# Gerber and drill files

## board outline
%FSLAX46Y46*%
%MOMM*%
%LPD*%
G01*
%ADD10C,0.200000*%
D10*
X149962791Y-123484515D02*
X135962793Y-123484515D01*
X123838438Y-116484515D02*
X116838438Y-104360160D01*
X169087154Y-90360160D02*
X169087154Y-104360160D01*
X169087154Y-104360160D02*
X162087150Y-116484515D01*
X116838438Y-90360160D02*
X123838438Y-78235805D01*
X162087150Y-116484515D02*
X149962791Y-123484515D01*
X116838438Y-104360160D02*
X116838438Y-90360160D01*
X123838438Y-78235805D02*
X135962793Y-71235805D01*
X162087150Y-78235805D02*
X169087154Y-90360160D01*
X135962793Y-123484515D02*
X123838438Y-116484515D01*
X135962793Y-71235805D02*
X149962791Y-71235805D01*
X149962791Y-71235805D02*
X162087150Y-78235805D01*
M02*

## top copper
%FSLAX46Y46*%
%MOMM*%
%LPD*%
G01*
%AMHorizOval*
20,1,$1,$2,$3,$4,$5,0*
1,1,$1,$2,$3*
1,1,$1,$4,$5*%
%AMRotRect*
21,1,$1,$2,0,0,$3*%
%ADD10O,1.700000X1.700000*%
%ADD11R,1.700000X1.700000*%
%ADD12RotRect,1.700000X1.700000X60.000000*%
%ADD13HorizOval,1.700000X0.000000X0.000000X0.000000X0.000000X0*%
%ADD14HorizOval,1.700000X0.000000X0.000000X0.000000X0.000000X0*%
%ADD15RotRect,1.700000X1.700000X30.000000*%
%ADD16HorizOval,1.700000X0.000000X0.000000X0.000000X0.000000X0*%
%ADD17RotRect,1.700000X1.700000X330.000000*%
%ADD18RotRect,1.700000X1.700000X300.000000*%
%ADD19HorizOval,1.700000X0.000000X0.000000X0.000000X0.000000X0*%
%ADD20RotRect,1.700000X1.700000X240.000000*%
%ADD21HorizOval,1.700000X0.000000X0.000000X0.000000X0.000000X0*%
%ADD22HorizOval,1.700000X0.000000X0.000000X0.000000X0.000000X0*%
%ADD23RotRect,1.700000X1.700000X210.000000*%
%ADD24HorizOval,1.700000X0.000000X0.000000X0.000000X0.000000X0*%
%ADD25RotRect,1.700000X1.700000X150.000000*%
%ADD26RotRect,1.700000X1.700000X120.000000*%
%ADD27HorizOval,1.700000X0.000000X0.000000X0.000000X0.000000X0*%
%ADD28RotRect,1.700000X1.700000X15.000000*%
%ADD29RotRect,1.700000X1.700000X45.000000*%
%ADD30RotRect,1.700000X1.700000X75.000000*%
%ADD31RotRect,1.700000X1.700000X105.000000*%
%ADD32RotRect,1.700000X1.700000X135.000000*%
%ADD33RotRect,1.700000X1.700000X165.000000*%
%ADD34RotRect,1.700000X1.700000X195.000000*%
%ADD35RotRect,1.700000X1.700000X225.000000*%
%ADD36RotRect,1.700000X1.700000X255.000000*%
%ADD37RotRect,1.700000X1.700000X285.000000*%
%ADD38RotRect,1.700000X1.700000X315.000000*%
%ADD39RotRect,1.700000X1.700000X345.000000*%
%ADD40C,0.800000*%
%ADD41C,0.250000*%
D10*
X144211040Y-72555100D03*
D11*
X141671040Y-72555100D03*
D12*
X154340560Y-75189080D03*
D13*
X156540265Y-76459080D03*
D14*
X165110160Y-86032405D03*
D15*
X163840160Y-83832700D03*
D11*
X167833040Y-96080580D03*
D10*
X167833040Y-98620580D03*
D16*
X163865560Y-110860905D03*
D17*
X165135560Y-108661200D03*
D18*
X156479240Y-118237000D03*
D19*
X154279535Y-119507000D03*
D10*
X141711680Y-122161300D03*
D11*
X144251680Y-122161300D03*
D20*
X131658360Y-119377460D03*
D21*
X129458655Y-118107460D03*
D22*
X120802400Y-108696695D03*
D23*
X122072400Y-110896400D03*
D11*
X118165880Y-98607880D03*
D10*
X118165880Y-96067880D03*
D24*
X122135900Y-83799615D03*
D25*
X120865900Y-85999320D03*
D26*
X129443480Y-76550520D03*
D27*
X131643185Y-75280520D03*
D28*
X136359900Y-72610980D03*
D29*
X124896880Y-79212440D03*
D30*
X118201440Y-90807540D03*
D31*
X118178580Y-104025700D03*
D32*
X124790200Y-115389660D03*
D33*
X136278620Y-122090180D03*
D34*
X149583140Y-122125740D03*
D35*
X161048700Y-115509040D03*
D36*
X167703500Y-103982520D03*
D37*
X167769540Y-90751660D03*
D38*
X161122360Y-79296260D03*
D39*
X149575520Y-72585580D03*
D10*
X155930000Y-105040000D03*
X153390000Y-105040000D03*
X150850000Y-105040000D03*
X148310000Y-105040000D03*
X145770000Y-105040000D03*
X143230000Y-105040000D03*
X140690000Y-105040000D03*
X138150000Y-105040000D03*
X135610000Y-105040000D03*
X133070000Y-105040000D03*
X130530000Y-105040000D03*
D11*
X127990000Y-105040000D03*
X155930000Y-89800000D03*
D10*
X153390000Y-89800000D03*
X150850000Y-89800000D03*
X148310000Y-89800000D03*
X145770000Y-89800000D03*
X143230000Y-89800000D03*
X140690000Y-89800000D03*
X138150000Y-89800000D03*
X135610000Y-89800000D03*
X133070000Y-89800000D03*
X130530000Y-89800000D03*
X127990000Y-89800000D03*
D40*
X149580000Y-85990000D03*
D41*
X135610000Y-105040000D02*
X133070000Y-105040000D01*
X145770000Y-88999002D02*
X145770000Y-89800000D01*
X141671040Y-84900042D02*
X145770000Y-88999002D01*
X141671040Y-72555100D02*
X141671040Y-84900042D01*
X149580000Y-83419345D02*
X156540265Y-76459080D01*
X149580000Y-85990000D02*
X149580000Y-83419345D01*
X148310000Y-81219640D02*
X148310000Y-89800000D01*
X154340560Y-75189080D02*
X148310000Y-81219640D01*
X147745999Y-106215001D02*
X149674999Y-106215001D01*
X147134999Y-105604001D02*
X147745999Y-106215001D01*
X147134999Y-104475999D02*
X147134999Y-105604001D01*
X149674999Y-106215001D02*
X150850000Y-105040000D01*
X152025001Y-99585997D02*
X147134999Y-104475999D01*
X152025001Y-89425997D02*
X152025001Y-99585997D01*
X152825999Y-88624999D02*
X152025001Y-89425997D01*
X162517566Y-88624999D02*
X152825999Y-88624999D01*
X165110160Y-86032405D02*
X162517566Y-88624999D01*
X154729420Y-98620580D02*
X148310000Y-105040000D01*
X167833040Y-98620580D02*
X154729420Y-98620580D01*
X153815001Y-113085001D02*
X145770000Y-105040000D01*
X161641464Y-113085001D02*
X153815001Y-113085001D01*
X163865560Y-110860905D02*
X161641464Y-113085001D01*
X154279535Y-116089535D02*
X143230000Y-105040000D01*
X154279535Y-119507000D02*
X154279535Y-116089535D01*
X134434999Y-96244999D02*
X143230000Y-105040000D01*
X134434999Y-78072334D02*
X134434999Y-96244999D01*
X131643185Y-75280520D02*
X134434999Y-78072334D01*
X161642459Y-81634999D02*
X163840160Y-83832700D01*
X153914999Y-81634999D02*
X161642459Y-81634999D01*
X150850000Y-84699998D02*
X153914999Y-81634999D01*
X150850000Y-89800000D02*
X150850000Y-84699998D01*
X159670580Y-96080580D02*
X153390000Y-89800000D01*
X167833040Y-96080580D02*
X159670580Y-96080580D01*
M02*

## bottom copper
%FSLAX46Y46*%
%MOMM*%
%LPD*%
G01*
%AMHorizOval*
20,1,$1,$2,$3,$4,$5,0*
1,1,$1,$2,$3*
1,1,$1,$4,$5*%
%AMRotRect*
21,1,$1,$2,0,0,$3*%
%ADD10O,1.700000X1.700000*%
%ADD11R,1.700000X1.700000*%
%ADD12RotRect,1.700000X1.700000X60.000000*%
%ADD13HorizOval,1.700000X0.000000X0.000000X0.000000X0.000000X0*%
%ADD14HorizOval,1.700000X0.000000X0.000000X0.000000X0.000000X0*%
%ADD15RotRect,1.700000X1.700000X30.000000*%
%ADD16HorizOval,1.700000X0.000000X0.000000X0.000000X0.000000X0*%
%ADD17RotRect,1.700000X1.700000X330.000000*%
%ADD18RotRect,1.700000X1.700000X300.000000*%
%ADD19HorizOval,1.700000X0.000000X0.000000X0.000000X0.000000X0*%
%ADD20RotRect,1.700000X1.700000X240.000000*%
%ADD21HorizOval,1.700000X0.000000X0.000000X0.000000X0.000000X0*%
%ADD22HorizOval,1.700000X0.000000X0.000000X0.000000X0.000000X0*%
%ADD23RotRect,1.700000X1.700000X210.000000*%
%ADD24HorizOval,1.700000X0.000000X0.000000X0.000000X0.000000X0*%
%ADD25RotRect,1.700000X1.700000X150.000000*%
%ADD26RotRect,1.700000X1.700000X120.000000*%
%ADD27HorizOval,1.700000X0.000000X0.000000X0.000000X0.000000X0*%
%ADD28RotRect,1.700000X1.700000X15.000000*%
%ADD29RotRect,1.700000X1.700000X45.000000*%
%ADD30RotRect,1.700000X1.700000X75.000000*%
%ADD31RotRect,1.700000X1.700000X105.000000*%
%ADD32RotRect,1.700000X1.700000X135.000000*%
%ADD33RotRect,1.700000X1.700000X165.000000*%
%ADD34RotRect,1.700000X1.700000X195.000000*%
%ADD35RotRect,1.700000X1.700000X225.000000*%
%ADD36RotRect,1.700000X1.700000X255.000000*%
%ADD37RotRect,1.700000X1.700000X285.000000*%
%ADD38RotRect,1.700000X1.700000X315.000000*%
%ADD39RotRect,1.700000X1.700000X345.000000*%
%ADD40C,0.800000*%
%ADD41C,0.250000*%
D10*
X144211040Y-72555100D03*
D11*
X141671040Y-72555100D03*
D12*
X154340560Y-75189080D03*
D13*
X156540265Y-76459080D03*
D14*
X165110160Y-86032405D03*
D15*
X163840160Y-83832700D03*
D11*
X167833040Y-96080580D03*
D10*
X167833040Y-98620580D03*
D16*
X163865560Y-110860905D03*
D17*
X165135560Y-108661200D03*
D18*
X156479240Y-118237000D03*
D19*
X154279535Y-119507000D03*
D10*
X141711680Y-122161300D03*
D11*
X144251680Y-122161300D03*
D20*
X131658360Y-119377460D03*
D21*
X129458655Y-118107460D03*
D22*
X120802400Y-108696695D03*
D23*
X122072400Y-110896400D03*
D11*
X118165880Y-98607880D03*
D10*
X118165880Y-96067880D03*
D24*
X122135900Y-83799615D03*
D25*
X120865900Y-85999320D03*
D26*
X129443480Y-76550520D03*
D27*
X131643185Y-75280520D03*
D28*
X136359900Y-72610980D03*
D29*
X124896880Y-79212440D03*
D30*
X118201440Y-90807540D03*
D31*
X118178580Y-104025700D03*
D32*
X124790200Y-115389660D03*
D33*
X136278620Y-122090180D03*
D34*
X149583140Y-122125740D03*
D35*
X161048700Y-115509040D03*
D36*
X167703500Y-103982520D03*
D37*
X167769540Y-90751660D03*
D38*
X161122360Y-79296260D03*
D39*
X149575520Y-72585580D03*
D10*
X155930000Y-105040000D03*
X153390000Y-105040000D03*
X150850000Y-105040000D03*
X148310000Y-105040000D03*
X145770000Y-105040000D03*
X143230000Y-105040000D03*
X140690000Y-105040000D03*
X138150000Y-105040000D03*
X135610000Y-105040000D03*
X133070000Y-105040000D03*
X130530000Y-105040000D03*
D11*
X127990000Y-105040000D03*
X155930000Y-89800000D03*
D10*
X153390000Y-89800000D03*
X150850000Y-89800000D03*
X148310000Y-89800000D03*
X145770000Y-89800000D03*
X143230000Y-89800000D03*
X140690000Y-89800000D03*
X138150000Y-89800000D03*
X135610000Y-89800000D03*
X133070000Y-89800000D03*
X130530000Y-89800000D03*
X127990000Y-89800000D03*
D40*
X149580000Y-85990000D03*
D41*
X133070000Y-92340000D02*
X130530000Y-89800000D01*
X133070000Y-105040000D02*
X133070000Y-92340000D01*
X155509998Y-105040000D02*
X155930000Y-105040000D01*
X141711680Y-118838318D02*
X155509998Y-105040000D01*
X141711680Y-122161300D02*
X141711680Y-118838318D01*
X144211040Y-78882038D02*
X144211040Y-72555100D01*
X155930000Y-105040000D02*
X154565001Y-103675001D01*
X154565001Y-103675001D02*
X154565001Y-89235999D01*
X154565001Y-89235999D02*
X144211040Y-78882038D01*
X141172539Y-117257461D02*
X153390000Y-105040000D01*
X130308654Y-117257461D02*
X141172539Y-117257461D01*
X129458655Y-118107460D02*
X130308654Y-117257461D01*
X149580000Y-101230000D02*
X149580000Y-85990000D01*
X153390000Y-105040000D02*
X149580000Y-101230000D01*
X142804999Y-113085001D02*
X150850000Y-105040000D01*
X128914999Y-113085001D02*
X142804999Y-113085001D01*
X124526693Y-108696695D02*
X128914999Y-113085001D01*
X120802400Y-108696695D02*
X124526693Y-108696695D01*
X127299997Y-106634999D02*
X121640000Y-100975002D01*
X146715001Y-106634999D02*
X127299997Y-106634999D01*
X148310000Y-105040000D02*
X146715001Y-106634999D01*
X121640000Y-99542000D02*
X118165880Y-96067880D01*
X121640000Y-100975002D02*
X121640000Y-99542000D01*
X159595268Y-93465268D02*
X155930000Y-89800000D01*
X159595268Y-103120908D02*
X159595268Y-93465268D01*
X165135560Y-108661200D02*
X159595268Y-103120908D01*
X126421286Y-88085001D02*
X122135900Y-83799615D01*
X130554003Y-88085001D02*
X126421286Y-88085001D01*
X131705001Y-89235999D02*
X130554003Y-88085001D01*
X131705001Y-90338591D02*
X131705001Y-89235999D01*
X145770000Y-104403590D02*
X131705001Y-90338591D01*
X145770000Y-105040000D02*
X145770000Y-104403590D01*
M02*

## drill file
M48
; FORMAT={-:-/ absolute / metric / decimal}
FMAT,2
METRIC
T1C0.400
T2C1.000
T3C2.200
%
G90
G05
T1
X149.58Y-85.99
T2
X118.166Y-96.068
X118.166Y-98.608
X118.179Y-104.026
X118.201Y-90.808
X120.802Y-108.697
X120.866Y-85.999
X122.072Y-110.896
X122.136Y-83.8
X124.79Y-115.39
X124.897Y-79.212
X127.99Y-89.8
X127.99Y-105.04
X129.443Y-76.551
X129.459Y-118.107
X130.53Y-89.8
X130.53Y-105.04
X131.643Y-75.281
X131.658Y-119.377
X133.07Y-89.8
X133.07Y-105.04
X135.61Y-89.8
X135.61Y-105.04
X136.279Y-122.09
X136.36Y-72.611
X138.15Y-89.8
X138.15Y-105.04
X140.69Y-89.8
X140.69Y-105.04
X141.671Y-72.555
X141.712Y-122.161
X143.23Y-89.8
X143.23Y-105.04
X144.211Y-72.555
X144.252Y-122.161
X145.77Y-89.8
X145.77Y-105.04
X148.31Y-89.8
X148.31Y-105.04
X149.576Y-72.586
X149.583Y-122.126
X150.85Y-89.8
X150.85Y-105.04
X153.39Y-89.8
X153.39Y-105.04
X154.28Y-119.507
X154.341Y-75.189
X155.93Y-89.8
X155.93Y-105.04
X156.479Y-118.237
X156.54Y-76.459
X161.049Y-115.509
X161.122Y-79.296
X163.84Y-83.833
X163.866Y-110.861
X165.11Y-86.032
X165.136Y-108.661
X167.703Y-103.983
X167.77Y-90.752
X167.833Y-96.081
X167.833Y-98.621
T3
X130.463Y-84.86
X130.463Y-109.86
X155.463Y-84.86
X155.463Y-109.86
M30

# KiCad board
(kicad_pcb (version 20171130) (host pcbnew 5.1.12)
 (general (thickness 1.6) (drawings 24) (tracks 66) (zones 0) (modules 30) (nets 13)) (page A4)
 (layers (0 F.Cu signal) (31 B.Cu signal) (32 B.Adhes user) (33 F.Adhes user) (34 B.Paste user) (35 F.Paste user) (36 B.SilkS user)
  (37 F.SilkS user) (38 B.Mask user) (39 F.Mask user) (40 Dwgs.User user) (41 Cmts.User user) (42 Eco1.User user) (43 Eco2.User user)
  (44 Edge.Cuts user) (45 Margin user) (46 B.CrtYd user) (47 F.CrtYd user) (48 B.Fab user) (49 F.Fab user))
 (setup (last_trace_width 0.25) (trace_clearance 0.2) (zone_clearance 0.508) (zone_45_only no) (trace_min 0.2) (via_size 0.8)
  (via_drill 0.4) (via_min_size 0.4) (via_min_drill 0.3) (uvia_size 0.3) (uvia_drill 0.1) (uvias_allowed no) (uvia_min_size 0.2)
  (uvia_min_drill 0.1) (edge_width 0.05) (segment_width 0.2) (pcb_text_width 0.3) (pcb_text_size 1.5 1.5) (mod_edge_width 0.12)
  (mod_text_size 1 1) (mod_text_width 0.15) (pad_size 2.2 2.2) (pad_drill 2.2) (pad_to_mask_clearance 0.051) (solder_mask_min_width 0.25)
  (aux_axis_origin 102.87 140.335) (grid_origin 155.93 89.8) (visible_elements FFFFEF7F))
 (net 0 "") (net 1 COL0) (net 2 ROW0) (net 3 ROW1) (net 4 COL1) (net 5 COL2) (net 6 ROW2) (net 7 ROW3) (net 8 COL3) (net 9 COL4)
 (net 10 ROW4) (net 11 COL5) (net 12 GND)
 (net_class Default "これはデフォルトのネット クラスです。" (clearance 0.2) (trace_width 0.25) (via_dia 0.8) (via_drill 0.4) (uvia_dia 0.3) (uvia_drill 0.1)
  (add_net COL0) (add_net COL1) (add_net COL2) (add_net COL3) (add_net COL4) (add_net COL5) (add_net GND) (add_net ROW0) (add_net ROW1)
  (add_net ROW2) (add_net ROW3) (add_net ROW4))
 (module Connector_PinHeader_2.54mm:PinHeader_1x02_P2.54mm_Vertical (layer F.Cu) (at 141.67104 72.5551 90)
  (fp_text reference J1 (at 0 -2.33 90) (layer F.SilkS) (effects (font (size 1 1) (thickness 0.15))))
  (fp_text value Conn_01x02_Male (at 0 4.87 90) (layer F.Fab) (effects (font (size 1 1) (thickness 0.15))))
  (pad 2 thru_hole oval (at 0 2.54 90) (size 1.7 1.7) (drill 1) (layers *.Cu *.Mask) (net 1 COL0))
  (pad 1 thru_hole rect (at 0 0 90) (size 1.7 1.7) (drill 1) (layers *.Cu *.Mask) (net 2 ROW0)))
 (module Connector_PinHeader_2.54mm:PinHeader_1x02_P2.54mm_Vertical (layer F.Cu) (at 154.34056 75.18908 60)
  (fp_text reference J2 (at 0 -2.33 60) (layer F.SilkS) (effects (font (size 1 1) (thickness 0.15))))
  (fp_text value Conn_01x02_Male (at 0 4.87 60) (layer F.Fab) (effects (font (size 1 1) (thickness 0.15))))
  (pad 1 thru_hole rect (at 0 0 60) (size 1.7 1.7) (drill 1) (layers *.Cu *.Mask) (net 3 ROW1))
  (pad 2 thru_hole oval (at 0 2.54 60) (size 1.7 1.7) (drill 1) (layers *.Cu *.Mask) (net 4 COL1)))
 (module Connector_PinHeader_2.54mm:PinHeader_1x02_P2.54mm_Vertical (layer F.Cu) (at 163.84016 83.8327 30)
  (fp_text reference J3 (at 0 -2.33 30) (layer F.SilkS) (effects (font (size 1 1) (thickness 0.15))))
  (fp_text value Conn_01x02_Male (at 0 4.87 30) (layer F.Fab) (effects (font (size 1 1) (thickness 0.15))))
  (pad 2 thru_hole oval (at 0 2.54 30) (size 1.7 1.7) (drill 1) (layers *.Cu *.Mask) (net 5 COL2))
  (pad 1 thru_hole rect (at 0 0 30) (size 1.7 1.7) (drill 1) (layers *.Cu *.Mask) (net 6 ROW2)))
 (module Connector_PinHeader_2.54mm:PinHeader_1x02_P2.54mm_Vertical (layer F.Cu) (at 167.83304 96.08058)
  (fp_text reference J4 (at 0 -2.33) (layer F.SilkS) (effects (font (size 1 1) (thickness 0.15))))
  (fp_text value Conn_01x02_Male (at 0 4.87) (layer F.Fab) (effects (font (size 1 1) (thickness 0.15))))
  (pad 1 thru_hole rect (at 0 0) (size 1.7 1.7) (drill 1) (layers *.Cu *.Mask) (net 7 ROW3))
  (pad 2 thru_hole oval (at 0 2.54) (size 1.7 1.7) (drill 1) (layers *.Cu *.Mask) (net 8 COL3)))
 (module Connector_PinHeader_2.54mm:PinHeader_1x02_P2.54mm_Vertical (layer F.Cu) (at 165.13556 108.6612 330)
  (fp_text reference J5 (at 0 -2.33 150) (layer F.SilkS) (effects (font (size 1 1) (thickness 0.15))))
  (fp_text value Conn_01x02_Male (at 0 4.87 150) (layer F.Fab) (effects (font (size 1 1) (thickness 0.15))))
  (pad 2 thru_hole oval (at 0 2.54 330) (size 1.7 1.7) (drill 1) (layers *.Cu *.Mask) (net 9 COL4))
  (pad 1 thru_hole rect (at 0 0 330) (size 1.7 1.7) (drill 1) (layers *.Cu *.Mask) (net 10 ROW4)))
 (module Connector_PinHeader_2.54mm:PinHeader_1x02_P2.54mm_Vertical (layer F.Cu) (at 156.47924 118.237 300)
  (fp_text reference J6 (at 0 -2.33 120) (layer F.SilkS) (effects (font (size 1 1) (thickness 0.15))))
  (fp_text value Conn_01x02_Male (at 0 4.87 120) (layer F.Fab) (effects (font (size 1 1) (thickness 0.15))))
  (pad 1 thru_hole rect (at 0 0 300) (size 1.7 1.7) (drill 1) (layers *.Cu *.Mask))
  (pad 2 thru_hole oval (at 0 2.54 300) (size 1.7 1.7) (drill 1) (layers *.Cu *.Mask) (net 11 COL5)))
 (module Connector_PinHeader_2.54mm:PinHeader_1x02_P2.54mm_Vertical (layer F.Cu) (at 144.25168 122.1613 270)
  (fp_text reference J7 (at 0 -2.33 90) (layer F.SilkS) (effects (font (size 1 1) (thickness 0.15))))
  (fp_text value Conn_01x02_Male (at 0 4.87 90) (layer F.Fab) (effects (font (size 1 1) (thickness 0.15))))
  (pad 2 thru_hole oval (at 0 2.54 270) (size 1.7 1.7) (drill 1) (layers *.Cu *.Mask) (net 1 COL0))
  (pad 1 thru_hole rect (at 0 0 270) (size 1.7 1.7) (drill 1) (layers *.Cu *.Mask)))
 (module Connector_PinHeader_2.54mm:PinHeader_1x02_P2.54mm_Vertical (layer F.Cu) (at 131.65836 119.37746 240)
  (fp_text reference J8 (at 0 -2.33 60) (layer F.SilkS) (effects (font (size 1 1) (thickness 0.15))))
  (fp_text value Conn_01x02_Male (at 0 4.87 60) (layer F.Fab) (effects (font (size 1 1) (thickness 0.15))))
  (pad 1 thru_hole rect (at 0 0 240) (size 1.7 1.7) (drill 1) (layers *.Cu *.Mask))
  (pad 2 thru_hole oval (at 0 2.54 240) (size 1.7 1.7) (drill 1) (layers *.Cu *.Mask) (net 4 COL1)))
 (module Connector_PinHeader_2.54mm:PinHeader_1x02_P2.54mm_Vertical (layer F.Cu) (at 122.0724 110.8964 210)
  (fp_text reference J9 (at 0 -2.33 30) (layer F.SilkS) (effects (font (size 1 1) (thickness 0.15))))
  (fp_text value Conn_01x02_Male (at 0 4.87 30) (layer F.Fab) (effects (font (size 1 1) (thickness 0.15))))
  (pad 2 thru_hole oval (at 0 2.54 210) (size 1.7 1.7) (drill 1) (layers *.Cu *.Mask) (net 5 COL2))
  (pad 1 thru_hole rect (at 0 0 210) (size 1.7 1.7) (drill 1) (layers *.Cu *.Mask)))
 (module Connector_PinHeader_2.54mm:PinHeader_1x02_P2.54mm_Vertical (layer F.Cu) (at 118.16588 98.60788 180)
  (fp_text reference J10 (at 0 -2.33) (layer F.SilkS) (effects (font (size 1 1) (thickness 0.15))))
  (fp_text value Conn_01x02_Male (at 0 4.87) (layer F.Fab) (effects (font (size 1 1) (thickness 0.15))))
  (pad 1 thru_hole rect (at 0 0 180) (size 1.7 1.7) (drill 1) (layers *.Cu *.Mask))
  (pad 2 thru_hole oval (at 0 2.54 180) (size 1.7 1.7) (drill 1) (layers *.Cu *.Mask) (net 8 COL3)))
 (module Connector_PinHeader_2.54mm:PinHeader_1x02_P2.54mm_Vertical (layer F.Cu) (at 120.8659 85.99932 150)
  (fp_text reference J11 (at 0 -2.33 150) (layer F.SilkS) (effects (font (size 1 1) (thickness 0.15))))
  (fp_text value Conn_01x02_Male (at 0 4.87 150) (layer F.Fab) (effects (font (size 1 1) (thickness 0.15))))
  (pad 2 thru_hole oval (at 0 2.54 150) (size 1.7 1.7) (drill 1) (layers *.Cu *.Mask) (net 9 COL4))
  (pad 1 thru_hole rect (at 0 0 150) (size 1.7 1.7) (drill 1) (layers *.Cu *.Mask)))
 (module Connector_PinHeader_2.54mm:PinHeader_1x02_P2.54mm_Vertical (layer F.Cu) (at 129.44348 76.55052 120)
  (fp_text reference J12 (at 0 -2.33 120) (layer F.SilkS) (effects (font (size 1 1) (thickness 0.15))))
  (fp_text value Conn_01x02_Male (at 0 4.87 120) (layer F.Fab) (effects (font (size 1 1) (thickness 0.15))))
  (pad 1 thru_hole rect (at 0 0 120) (size 1.7 1.7) (drill 1) (layers *.Cu *.Mask))
  (pad 2 thru_hole oval (at 0 2.54 120) (size 1.7 1.7) (drill 1) (layers *.Cu *.Mask) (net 11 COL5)))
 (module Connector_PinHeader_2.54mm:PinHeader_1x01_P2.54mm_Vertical (layer F.Cu) (at 136.3599 72.61098 15)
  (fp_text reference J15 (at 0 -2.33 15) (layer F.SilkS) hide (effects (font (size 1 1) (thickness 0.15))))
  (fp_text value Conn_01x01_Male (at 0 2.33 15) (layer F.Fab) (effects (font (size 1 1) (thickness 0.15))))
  (pad 1 thru_hole rect (at 0 0 15) (size 1.7 1.7) (drill 1) (layers *.Cu *.Mask)))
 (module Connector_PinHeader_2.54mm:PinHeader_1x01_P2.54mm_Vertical (layer F.Cu) (at 124.89688 79.21244 45)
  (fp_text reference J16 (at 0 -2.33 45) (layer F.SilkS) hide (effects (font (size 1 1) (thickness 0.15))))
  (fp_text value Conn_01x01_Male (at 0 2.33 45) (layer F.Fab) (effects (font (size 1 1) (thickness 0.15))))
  (pad 1 thru_hole rect (at 0 0 45) (size 1.7 1.7) (drill 1) (layers *.Cu *.Mask)))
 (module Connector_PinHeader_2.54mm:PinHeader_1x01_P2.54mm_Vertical (layer F.Cu) (at 118.20144 90.80754 75)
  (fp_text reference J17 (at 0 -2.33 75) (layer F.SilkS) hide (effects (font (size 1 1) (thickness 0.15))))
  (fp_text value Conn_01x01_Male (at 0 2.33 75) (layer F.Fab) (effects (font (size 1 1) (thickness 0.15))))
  (pad 1 thru_hole rect (at 0 0 75) (size 1.7 1.7) (drill 1) (layers *.Cu *.Mask)))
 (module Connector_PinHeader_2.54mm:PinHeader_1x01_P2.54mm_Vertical (layer F.Cu) (at 118.17858 104.0257 105)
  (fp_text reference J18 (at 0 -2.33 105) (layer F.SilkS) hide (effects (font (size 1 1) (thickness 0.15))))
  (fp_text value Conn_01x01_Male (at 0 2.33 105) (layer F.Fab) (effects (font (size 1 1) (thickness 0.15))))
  (pad 1 thru_hole rect (at 0 0 105) (size 1.7 1.7) (drill 1) (layers *.Cu *.Mask)))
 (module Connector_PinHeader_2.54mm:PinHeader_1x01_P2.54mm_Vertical (layer F.Cu) (at 124.7902 115.38966 135)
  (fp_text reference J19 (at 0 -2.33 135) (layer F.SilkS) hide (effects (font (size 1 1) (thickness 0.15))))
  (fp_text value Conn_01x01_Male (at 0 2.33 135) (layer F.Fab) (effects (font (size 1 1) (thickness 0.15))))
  (pad 1 thru_hole rect (at 0 0 135) (size 1.7 1.7) (drill 1) (layers *.Cu *.Mask)))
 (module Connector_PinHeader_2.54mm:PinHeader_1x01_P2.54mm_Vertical (layer F.Cu) (at 136.27862 122.09018 165)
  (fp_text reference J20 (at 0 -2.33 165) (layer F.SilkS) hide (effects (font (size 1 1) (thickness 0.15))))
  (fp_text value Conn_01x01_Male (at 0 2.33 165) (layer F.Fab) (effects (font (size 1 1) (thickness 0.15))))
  (pad 1 thru_hole rect (at 0 0 165) (size 1.7 1.7) (drill 1) (layers *.Cu *.Mask)))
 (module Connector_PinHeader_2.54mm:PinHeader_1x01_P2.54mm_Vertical (layer F.Cu) (at 149.58314 122.12574 195)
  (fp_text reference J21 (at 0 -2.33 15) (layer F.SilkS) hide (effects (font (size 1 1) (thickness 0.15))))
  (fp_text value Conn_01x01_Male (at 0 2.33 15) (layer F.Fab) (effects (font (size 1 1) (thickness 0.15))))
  (pad 1 thru_hole rect (at 0 0 195) (size 1.7 1.7) (drill 1) (layers *.Cu *.Mask)))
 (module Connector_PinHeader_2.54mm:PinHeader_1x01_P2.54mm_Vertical (layer F.Cu) (at 161.0487 115.50904 225)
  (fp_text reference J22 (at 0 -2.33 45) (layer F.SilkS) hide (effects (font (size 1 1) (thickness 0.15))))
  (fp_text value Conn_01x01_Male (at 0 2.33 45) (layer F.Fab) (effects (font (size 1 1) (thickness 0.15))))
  (pad 1 thru_hole rect (at 0 0 225) (size 1.7 1.7) (drill 1) (layers *.Cu *.Mask)))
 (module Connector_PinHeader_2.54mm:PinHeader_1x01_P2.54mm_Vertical (layer F.Cu) (at 167.7035 103.98252 255)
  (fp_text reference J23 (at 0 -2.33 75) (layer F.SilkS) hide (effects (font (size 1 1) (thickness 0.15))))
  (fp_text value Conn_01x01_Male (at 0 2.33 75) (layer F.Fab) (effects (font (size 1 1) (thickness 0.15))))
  (pad 1 thru_hole rect (at 0 0 255) (size 1.7 1.7) (drill 1) (layers *.Cu *.Mask)))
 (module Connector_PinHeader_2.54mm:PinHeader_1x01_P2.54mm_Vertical (layer F.Cu) (at 167.76954 90.75166 285)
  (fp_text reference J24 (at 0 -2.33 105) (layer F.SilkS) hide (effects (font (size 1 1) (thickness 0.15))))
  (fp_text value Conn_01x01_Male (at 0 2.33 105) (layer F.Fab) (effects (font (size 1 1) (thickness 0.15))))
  (pad 1 thru_hole rect (at 0 0 285) (size 1.7 1.7) (drill 1) (layers *.Cu *.Mask)))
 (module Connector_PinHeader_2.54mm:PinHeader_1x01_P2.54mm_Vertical (layer F.Cu) (at 161.12236 79.29626 315)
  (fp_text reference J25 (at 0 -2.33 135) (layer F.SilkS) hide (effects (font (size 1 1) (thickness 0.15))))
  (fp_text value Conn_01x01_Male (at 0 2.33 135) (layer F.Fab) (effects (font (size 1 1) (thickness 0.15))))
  (pad 1 thru_hole rect (at 0 0 315) (size 1.7 1.7) (drill 1) (layers *.Cu *.Mask)))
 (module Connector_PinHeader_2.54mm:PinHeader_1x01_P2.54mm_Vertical (layer F.Cu) (at 149.57552 72.58558 345)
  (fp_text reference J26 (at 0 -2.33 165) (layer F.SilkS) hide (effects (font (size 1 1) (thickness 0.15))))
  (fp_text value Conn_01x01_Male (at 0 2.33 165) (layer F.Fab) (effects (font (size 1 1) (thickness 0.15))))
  (pad 1 thru_hole rect (at 0 0 345) (size 1.7 1.7) (drill 1) (layers *.Cu *.Mask)))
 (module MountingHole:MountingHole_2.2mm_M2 (layer F.Cu) (at 155.463 109.86) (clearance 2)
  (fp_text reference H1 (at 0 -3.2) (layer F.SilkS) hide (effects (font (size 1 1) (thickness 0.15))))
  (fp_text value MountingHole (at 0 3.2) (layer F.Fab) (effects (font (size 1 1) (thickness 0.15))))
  (pad 1 np_thru_hole circle (at 0 0) (size 2.2 2.2) (drill 2.2) (layers *.Cu *.Mask)))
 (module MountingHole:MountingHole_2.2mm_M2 (layer F.Cu) (at 155.463 84.86) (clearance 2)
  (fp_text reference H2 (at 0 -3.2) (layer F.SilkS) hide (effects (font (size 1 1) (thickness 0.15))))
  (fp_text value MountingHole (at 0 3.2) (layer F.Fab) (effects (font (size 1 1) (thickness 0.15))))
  (pad 1 np_thru_hole circle (at 0 0) (size 2.2 2.2) (drill 2.2) (layers *.Cu *.Mask)))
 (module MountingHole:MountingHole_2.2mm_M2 (layer F.Cu) (at 130.463 109.86)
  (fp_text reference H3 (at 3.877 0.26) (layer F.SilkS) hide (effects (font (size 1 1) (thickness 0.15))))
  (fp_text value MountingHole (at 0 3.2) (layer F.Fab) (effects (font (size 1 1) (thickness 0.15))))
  (pad "" np_thru_hole circle (at 0 0) (size 2.2 2.2) (drill 2.2) (layers *.Cu *.Mask) (clearance 2)))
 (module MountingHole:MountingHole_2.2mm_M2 (layer F.Cu) (at 130.463 84.86) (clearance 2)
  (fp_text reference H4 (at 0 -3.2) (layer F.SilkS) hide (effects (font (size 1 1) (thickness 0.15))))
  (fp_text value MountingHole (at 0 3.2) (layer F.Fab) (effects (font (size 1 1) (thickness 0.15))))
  (pad 1 np_thru_hole circle (at 0 0) (size 2.2 2.2) (drill 2.2) (layers *.Cu *.Mask)))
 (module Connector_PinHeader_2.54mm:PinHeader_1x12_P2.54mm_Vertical (layer F.Cu) (at 127.99 105.04 90)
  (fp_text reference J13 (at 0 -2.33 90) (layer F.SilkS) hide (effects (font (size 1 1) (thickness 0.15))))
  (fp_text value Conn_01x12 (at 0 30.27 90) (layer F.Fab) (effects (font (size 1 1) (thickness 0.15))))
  (pad 12 thru_hole oval (at 0 27.94 90) (size 1.7 1.7) (drill 1) (layers *.Cu *.Mask) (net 1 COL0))
  (pad 11 thru_hole oval (at 0 25.4 90) (size 1.7 1.7) (drill 1) (layers *.Cu *.Mask) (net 4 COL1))
  (pad 10 thru_hole oval (at 0 22.86 90) (size 1.7 1.7) (drill 1) (layers *.Cu *.Mask) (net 5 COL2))
  (pad 9 thru_hole oval (at 0 20.32 90) (size 1.7 1.7) (drill 1) (layers *.Cu *.Mask) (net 8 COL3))
  (pad 8 thru_hole oval (at 0 17.78 90) (size 1.7 1.7) (drill 1) (layers *.Cu *.Mask) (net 9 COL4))
  (pad 7 thru_hole oval (at 0 15.24 90) (size 1.7 1.7) (drill 1) (layers *.Cu *.Mask) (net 11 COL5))
  (pad 6 thru_hole oval (at 0 12.7 90) (size 1.7 1.7) (drill 1) (layers *.Cu *.Mask))
  (pad 5 thru_hole oval (at 0 10.16 90) (size 1.7 1.7) (drill 1) (layers *.Cu *.Mask))
  (pad 4 thru_hole oval (at 0 7.62 90) (size 1.7 1.7) (drill 1) (layers *.Cu *.Mask) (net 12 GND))
  (pad 3 thru_hole oval (at 0 5.08 90) (size 1.7 1.7) (drill 1) (layers *.Cu *.Mask) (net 12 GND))
  (pad 2 thru_hole oval (at 0 2.54 90) (size 1.7 1.7) (drill 1) (layers *.Cu *.Mask))
  (pad 1 thru_hole rect (at 0 0 90) (size 1.7 1.7) (drill 1) (layers *.Cu *.Mask)))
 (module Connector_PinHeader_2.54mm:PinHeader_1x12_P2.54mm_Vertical (layer F.Cu) (at 155.93 89.8 270)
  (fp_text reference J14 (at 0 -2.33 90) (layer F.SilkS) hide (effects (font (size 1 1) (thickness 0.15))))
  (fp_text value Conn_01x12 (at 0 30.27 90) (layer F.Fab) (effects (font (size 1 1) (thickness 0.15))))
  (pad 1 thru_hole rect (at 0 0 270) (size 1.7 1.7) (drill 1) (layers *.Cu *.Mask) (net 10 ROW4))
  (pad 2 thru_hole oval (at 0 2.54 270) (size 1.7 1.7) (drill 1) (layers *.Cu *.Mask) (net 7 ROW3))
  (pad 3 thru_hole oval (at 0 5.08 270) (size 1.7 1.7) (drill 1) (layers *.Cu *.Mask) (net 6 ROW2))
  (pad 4 thru_hole oval (at 0 7.62 270) (size 1.7 1.7) (drill 1) (layers *.Cu *.Mask) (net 3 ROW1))
  (pad 5 thru_hole oval (at 0 10.16 270) (size 1.7 1.7) (drill 1) (layers *.Cu *.Mask) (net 2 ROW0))
  (pad 6 thru_hole oval (at 0 12.7 270) (size 1.7 1.7) (drill 1) (layers *.Cu *.Mask))
  (pad 7 thru_hole oval (at 0 15.24 270) (size 1.7 1.7) (drill 1) (layers *.Cu *.Mask))
  (pad 8 thru_hole oval (at 0 17.78 270) (size 1.7 1.7) (drill 1) (layers *.Cu *.Mask))
  (pad 9 thru_hole oval (at 0 20.32 270) (size 1.7 1.7) (drill 1) (layers *.Cu *.Mask))
  (pad 10 thru_hole oval (at 0 22.86 270) (size 1.7 1.7) (drill 1) (layers *.Cu *.Mask))
  (pad 11 thru_hole oval (at 0 25.4 270) (size 1.7 1.7) (drill 1) (layers *.Cu *.Mask) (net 12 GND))
  (pad 12 thru_hole oval (at 0 27.94 270) (size 1.7 1.7) (drill 1) (layers *.Cu *.Mask)))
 (gr_line (start 149.962791 123.484515) (end 135.962793 123.484515) (layer Edge.Cuts) (width 0.2))
 (gr_line (start 123.838438 116.484515) (end 116.838438 104.36016) (layer Edge.Cuts) (width 0.2))
 (gr_line (start 169.087154 90.36016) (end 169.087154 104.36016) (layer Edge.Cuts) (width 0.2))
 (gr_line (start 169.087154 104.36016) (end 162.08715 116.484515) (layer Edge.Cuts) (width 0.2))
 (gr_line (start 116.838438 90.36016) (end 123.838438 78.235805) (layer Edge.Cuts) (width 0.2))
 (gr_line (start 162.08715 116.484515) (end 149.962791 123.484515) (layer Edge.Cuts) (width 0.2))
 (gr_line (start 116.838438 104.36016) (end 116.838438 90.36016) (layer Edge.Cuts) (width 0.2))
 (gr_line (start 123.838438 78.235805) (end 135.962793 71.235805) (layer Edge.Cuts) (width 0.2))
 (gr_line (start 162.08715 78.235805) (end 169.087154 90.36016) (layer Edge.Cuts) (width 0.2))
 (gr_line (start 135.962793 123.484515) (end 123.838438 116.484515) (layer Edge.Cuts) (width 0.2))
 (gr_line (start 135.962793 71.235805) (end 149.962791 71.235805) (layer Edge.Cuts) (width 0.2))
 (gr_line (start 149.962791 71.235805) (end 162.08715 78.235805) (layer Edge.Cuts) (width 0.2))
 (segment (start 135.61 105.04) (end 133.07 105.04) (width 0.25) (layer F.Cu) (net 12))
 (segment (start 133.07 92.34) (end 130.53 89.8) (width 0.25) (layer B.Cu) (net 12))
 (segment (start 133.07 105.04) (end 133.07 92.34) (width 0.25) (layer B.Cu) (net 12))
 (segment (start 145.77 88.999002) (end 145.77 89.8) (width 0.25) (layer F.Cu) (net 2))
 (segment (start 141.67104 84.900042) (end 145.77 88.999002) (width 0.25) (layer F.Cu) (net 2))
 (segment (start 141.67104 72.5551) (end 141.67104 84.900042) (width 0.25) (layer F.Cu) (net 2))
 (segment (start 155.509998 105.04) (end 155.93 105.04) (width 0.25) (layer B.Cu) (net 1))
 (segment (start 141.71168 118.838318) (end 155.509998 105.04) (width 0.25) (layer B.Cu) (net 1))
 (segment (start 141.71168 122.1613) (end 141.71168 118.838318) (width 0.25) (layer B.Cu) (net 1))
 (segment (start 144.21104 78.882038) (end 144.21104 72.5551) (width 0.25) (layer B.Cu) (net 1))
 (segment (start 155.93 105.04) (end 154.565001 103.675001) (width 0.25) (layer B.Cu) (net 1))
 (segment (start 154.565001 103.675001) (end 154.565001 89.235999) (width 0.25) (layer B.Cu) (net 1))
 (segment (start 154.565001 89.235999) (end 144.21104 78.882038) (width 0.25) (layer B.Cu) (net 1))
 (segment (start 141.172539 117.257461) (end 153.39 105.04) (width 0.25) (layer B.Cu) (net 4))
 (segment (start 130.308654 117.257461) (end 141.172539 117.257461) (width 0.25) (layer B.Cu) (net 4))
 (segment (start 129.458655 118.10746) (end 130.308654 117.257461) (width 0.25) (layer B.Cu) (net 4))
 (via (at 149.58 85.99) (size 0.8) (drill 0.4) (layers F.Cu B.Cu) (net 4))
 (segment (start 149.58 101.23) (end 149.58 85.99) (width 0.25) (layer B.Cu) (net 4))
 (segment (start 153.39 105.04) (end 149.58 101.23) (width 0.25) (layer B.Cu) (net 4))
 (segment (start 149.58 83.419345) (end 156.540265 76.45908) (width 0.25) (layer F.Cu) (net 4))
 (segment (start 149.58 85.99) (end 149.58 83.419345) (width 0.25) (layer F.Cu) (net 4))
 (segment (start 148.31 81.21964) (end 148.31 89.8) (width 0.25) (layer F.Cu) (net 3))
 (segment (start 154.34056 75.18908) (end 148.31 81.21964) (width 0.25) (layer F.Cu) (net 3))
 (segment (start 142.804999 113.085001) (end 150.85 105.04) (width 0.25) (layer B.Cu) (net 5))
 (segment (start 128.914999 113.085001) (end 142.804999 113.085001) (width 0.25) (layer B.Cu) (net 5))
 (segment (start 124.526693 108.696695) (end 128.914999 113.085001) (width 0.25) (layer B.Cu) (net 5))
 (segment (start 120.8024 108.696695) (end 124.526693 108.696695) (width 0.25) (layer B.Cu) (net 5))
 (segment (start 147.745999 106.215001) (end 149.674999 106.215001) (width 0.25) (layer F.Cu) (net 5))
 (segment (start 147.134999 105.604001) (end 147.745999 106.215001) (width 0.25) (layer F.Cu) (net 5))
 (segment (start 147.134999 104.475999) (end 147.134999 105.604001) (width 0.25) (layer F.Cu) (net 5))
 (segment (start 149.674999 106.215001) (end 150.85 105.04) (width 0.25) (layer F.Cu) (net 5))
 (segment (start 152.025001 99.585997) (end 147.134999 104.475999) (width 0.25) (layer F.Cu) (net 5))
 (segment (start 152.025001 89.425997) (end 152.025001 99.585997) (width 0.25) (layer F.Cu) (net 5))
 (segment (start 152.825999 88.624999) (end 152.025001 89.425997) (width 0.25) (layer F.Cu) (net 5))
 (segment (start 162.517566 88.624999) (end 152.825999 88.624999) (width 0.25) (layer F.Cu) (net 5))
 (segment (start 165.11016 86.032405) (end 162.517566 88.624999) (width 0.25) (layer F.Cu) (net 5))
 (segment (start 154.72942 98.62058) (end 148.31 105.04) (width 0.25) (layer F.Cu) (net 8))
 (segment (start 167.83304 98.62058) (end 154.72942 98.62058) (width 0.25) (layer F.Cu) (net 8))
 (segment (start 127.299997 106.634999) (end 121.64 100.975002) (width 0.25) (layer B.Cu) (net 8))
 (segment (start 146.715001 106.634999) (end 127.299997 106.634999) (width 0.25) (layer B.Cu) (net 8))
 (segment (start 148.31 105.04) (end 146.715001 106.634999) (width 0.25) (layer B.Cu) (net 8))
 (segment (start 121.64 99.542) (end 118.16588 96.06788) (width 0.25) (layer B.Cu) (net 8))
 (segment (start 121.64 100.975002) (end 121.64 99.542) (width 0.25) (layer B.Cu) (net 8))
 (segment (start 159.595268 93.465268) (end 155.93 89.8) (width 0.25) (layer B.Cu) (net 10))
 (segment (start 159.595268 103.120908) (end 159.595268 93.465268) (width 0.25) (layer B.Cu) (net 10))
 (segment (start 165.13556 108.6612) (end 159.595268 103.120908) (width 0.25) (layer B.Cu) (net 10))
 (segment (start 126.421286 88.085001) (end 122.1359 83.799615) (width 0.25) (layer B.Cu) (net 9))
 (segment (start 130.554003 88.085001) (end 126.421286 88.085001) (width 0.25) (layer B.Cu) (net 9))
 (segment (start 131.705001 89.235999) (end 130.554003 88.085001) (width 0.25) (layer B.Cu) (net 9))
 (segment (start 131.705001 90.338591) (end 131.705001 89.235999) (width 0.25) (layer B.Cu) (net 9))
 (segment (start 145.77 104.40359) (end 131.705001 90.338591) (width 0.25) (layer B.Cu) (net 9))
 (segment (start 145.77 105.04) (end 145.77 104.40359) (width 0.25) (layer B.Cu) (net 9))
 (segment (start 153.815001 113.085001) (end 145.77 105.04) (width 0.25) (layer F.Cu) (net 9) (status 1000000))
 (segment (start 161.641464 113.085001) (end 153.815001 113.085001) (width 0.25) (layer F.Cu) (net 9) (status 1000000))
 (segment (start 163.86556 110.860905) (end 161.641464 113.085001) (width 0.25) (layer F.Cu) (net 9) (status 1000000))
 (segment (start 154.279535 116.089535) (end 143.23 105.04) (width 0.25) (layer F.Cu) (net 11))
 (segment (start 154.279535 119.507) (end 154.279535 116.089535) (width 0.25) (layer F.Cu) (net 11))
 (segment (start 134.434999 96.244999) (end 143.23 105.04) (width 0.25) (layer F.Cu) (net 11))
 (segment (start 134.434999 78.072334) (end 134.434999 96.244999) (width 0.25) (layer F.Cu) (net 11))
 (segment (start 131.643185 75.28052) (end 134.434999 78.072334) (width 0.25) (layer F.Cu) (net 11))
 (segment (start 161.642459 81.634999) (end 163.84016 83.8327) (width 0.25) (layer F.Cu) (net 6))
 (segment (start 153.914999 81.634999) (end 161.642459 81.634999) (width 0.25) (layer F.Cu) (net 6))
 (segment (start 150.85 84.699998) (end 153.914999 81.634999) (width 0.25) (layer F.Cu) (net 6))
 (segment (start 150.85 89.8) (end 150.85 84.699998) (width 0.25) (layer F.Cu) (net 6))
 (segment (start 159.67058 96.08058) (end 153.39 89.8) (width 0.25) (layer F.Cu) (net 7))
 (segment (start 167.83304 96.08058) (end 159.67058 96.08058) (width 0.25) (layer F.Cu) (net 7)))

